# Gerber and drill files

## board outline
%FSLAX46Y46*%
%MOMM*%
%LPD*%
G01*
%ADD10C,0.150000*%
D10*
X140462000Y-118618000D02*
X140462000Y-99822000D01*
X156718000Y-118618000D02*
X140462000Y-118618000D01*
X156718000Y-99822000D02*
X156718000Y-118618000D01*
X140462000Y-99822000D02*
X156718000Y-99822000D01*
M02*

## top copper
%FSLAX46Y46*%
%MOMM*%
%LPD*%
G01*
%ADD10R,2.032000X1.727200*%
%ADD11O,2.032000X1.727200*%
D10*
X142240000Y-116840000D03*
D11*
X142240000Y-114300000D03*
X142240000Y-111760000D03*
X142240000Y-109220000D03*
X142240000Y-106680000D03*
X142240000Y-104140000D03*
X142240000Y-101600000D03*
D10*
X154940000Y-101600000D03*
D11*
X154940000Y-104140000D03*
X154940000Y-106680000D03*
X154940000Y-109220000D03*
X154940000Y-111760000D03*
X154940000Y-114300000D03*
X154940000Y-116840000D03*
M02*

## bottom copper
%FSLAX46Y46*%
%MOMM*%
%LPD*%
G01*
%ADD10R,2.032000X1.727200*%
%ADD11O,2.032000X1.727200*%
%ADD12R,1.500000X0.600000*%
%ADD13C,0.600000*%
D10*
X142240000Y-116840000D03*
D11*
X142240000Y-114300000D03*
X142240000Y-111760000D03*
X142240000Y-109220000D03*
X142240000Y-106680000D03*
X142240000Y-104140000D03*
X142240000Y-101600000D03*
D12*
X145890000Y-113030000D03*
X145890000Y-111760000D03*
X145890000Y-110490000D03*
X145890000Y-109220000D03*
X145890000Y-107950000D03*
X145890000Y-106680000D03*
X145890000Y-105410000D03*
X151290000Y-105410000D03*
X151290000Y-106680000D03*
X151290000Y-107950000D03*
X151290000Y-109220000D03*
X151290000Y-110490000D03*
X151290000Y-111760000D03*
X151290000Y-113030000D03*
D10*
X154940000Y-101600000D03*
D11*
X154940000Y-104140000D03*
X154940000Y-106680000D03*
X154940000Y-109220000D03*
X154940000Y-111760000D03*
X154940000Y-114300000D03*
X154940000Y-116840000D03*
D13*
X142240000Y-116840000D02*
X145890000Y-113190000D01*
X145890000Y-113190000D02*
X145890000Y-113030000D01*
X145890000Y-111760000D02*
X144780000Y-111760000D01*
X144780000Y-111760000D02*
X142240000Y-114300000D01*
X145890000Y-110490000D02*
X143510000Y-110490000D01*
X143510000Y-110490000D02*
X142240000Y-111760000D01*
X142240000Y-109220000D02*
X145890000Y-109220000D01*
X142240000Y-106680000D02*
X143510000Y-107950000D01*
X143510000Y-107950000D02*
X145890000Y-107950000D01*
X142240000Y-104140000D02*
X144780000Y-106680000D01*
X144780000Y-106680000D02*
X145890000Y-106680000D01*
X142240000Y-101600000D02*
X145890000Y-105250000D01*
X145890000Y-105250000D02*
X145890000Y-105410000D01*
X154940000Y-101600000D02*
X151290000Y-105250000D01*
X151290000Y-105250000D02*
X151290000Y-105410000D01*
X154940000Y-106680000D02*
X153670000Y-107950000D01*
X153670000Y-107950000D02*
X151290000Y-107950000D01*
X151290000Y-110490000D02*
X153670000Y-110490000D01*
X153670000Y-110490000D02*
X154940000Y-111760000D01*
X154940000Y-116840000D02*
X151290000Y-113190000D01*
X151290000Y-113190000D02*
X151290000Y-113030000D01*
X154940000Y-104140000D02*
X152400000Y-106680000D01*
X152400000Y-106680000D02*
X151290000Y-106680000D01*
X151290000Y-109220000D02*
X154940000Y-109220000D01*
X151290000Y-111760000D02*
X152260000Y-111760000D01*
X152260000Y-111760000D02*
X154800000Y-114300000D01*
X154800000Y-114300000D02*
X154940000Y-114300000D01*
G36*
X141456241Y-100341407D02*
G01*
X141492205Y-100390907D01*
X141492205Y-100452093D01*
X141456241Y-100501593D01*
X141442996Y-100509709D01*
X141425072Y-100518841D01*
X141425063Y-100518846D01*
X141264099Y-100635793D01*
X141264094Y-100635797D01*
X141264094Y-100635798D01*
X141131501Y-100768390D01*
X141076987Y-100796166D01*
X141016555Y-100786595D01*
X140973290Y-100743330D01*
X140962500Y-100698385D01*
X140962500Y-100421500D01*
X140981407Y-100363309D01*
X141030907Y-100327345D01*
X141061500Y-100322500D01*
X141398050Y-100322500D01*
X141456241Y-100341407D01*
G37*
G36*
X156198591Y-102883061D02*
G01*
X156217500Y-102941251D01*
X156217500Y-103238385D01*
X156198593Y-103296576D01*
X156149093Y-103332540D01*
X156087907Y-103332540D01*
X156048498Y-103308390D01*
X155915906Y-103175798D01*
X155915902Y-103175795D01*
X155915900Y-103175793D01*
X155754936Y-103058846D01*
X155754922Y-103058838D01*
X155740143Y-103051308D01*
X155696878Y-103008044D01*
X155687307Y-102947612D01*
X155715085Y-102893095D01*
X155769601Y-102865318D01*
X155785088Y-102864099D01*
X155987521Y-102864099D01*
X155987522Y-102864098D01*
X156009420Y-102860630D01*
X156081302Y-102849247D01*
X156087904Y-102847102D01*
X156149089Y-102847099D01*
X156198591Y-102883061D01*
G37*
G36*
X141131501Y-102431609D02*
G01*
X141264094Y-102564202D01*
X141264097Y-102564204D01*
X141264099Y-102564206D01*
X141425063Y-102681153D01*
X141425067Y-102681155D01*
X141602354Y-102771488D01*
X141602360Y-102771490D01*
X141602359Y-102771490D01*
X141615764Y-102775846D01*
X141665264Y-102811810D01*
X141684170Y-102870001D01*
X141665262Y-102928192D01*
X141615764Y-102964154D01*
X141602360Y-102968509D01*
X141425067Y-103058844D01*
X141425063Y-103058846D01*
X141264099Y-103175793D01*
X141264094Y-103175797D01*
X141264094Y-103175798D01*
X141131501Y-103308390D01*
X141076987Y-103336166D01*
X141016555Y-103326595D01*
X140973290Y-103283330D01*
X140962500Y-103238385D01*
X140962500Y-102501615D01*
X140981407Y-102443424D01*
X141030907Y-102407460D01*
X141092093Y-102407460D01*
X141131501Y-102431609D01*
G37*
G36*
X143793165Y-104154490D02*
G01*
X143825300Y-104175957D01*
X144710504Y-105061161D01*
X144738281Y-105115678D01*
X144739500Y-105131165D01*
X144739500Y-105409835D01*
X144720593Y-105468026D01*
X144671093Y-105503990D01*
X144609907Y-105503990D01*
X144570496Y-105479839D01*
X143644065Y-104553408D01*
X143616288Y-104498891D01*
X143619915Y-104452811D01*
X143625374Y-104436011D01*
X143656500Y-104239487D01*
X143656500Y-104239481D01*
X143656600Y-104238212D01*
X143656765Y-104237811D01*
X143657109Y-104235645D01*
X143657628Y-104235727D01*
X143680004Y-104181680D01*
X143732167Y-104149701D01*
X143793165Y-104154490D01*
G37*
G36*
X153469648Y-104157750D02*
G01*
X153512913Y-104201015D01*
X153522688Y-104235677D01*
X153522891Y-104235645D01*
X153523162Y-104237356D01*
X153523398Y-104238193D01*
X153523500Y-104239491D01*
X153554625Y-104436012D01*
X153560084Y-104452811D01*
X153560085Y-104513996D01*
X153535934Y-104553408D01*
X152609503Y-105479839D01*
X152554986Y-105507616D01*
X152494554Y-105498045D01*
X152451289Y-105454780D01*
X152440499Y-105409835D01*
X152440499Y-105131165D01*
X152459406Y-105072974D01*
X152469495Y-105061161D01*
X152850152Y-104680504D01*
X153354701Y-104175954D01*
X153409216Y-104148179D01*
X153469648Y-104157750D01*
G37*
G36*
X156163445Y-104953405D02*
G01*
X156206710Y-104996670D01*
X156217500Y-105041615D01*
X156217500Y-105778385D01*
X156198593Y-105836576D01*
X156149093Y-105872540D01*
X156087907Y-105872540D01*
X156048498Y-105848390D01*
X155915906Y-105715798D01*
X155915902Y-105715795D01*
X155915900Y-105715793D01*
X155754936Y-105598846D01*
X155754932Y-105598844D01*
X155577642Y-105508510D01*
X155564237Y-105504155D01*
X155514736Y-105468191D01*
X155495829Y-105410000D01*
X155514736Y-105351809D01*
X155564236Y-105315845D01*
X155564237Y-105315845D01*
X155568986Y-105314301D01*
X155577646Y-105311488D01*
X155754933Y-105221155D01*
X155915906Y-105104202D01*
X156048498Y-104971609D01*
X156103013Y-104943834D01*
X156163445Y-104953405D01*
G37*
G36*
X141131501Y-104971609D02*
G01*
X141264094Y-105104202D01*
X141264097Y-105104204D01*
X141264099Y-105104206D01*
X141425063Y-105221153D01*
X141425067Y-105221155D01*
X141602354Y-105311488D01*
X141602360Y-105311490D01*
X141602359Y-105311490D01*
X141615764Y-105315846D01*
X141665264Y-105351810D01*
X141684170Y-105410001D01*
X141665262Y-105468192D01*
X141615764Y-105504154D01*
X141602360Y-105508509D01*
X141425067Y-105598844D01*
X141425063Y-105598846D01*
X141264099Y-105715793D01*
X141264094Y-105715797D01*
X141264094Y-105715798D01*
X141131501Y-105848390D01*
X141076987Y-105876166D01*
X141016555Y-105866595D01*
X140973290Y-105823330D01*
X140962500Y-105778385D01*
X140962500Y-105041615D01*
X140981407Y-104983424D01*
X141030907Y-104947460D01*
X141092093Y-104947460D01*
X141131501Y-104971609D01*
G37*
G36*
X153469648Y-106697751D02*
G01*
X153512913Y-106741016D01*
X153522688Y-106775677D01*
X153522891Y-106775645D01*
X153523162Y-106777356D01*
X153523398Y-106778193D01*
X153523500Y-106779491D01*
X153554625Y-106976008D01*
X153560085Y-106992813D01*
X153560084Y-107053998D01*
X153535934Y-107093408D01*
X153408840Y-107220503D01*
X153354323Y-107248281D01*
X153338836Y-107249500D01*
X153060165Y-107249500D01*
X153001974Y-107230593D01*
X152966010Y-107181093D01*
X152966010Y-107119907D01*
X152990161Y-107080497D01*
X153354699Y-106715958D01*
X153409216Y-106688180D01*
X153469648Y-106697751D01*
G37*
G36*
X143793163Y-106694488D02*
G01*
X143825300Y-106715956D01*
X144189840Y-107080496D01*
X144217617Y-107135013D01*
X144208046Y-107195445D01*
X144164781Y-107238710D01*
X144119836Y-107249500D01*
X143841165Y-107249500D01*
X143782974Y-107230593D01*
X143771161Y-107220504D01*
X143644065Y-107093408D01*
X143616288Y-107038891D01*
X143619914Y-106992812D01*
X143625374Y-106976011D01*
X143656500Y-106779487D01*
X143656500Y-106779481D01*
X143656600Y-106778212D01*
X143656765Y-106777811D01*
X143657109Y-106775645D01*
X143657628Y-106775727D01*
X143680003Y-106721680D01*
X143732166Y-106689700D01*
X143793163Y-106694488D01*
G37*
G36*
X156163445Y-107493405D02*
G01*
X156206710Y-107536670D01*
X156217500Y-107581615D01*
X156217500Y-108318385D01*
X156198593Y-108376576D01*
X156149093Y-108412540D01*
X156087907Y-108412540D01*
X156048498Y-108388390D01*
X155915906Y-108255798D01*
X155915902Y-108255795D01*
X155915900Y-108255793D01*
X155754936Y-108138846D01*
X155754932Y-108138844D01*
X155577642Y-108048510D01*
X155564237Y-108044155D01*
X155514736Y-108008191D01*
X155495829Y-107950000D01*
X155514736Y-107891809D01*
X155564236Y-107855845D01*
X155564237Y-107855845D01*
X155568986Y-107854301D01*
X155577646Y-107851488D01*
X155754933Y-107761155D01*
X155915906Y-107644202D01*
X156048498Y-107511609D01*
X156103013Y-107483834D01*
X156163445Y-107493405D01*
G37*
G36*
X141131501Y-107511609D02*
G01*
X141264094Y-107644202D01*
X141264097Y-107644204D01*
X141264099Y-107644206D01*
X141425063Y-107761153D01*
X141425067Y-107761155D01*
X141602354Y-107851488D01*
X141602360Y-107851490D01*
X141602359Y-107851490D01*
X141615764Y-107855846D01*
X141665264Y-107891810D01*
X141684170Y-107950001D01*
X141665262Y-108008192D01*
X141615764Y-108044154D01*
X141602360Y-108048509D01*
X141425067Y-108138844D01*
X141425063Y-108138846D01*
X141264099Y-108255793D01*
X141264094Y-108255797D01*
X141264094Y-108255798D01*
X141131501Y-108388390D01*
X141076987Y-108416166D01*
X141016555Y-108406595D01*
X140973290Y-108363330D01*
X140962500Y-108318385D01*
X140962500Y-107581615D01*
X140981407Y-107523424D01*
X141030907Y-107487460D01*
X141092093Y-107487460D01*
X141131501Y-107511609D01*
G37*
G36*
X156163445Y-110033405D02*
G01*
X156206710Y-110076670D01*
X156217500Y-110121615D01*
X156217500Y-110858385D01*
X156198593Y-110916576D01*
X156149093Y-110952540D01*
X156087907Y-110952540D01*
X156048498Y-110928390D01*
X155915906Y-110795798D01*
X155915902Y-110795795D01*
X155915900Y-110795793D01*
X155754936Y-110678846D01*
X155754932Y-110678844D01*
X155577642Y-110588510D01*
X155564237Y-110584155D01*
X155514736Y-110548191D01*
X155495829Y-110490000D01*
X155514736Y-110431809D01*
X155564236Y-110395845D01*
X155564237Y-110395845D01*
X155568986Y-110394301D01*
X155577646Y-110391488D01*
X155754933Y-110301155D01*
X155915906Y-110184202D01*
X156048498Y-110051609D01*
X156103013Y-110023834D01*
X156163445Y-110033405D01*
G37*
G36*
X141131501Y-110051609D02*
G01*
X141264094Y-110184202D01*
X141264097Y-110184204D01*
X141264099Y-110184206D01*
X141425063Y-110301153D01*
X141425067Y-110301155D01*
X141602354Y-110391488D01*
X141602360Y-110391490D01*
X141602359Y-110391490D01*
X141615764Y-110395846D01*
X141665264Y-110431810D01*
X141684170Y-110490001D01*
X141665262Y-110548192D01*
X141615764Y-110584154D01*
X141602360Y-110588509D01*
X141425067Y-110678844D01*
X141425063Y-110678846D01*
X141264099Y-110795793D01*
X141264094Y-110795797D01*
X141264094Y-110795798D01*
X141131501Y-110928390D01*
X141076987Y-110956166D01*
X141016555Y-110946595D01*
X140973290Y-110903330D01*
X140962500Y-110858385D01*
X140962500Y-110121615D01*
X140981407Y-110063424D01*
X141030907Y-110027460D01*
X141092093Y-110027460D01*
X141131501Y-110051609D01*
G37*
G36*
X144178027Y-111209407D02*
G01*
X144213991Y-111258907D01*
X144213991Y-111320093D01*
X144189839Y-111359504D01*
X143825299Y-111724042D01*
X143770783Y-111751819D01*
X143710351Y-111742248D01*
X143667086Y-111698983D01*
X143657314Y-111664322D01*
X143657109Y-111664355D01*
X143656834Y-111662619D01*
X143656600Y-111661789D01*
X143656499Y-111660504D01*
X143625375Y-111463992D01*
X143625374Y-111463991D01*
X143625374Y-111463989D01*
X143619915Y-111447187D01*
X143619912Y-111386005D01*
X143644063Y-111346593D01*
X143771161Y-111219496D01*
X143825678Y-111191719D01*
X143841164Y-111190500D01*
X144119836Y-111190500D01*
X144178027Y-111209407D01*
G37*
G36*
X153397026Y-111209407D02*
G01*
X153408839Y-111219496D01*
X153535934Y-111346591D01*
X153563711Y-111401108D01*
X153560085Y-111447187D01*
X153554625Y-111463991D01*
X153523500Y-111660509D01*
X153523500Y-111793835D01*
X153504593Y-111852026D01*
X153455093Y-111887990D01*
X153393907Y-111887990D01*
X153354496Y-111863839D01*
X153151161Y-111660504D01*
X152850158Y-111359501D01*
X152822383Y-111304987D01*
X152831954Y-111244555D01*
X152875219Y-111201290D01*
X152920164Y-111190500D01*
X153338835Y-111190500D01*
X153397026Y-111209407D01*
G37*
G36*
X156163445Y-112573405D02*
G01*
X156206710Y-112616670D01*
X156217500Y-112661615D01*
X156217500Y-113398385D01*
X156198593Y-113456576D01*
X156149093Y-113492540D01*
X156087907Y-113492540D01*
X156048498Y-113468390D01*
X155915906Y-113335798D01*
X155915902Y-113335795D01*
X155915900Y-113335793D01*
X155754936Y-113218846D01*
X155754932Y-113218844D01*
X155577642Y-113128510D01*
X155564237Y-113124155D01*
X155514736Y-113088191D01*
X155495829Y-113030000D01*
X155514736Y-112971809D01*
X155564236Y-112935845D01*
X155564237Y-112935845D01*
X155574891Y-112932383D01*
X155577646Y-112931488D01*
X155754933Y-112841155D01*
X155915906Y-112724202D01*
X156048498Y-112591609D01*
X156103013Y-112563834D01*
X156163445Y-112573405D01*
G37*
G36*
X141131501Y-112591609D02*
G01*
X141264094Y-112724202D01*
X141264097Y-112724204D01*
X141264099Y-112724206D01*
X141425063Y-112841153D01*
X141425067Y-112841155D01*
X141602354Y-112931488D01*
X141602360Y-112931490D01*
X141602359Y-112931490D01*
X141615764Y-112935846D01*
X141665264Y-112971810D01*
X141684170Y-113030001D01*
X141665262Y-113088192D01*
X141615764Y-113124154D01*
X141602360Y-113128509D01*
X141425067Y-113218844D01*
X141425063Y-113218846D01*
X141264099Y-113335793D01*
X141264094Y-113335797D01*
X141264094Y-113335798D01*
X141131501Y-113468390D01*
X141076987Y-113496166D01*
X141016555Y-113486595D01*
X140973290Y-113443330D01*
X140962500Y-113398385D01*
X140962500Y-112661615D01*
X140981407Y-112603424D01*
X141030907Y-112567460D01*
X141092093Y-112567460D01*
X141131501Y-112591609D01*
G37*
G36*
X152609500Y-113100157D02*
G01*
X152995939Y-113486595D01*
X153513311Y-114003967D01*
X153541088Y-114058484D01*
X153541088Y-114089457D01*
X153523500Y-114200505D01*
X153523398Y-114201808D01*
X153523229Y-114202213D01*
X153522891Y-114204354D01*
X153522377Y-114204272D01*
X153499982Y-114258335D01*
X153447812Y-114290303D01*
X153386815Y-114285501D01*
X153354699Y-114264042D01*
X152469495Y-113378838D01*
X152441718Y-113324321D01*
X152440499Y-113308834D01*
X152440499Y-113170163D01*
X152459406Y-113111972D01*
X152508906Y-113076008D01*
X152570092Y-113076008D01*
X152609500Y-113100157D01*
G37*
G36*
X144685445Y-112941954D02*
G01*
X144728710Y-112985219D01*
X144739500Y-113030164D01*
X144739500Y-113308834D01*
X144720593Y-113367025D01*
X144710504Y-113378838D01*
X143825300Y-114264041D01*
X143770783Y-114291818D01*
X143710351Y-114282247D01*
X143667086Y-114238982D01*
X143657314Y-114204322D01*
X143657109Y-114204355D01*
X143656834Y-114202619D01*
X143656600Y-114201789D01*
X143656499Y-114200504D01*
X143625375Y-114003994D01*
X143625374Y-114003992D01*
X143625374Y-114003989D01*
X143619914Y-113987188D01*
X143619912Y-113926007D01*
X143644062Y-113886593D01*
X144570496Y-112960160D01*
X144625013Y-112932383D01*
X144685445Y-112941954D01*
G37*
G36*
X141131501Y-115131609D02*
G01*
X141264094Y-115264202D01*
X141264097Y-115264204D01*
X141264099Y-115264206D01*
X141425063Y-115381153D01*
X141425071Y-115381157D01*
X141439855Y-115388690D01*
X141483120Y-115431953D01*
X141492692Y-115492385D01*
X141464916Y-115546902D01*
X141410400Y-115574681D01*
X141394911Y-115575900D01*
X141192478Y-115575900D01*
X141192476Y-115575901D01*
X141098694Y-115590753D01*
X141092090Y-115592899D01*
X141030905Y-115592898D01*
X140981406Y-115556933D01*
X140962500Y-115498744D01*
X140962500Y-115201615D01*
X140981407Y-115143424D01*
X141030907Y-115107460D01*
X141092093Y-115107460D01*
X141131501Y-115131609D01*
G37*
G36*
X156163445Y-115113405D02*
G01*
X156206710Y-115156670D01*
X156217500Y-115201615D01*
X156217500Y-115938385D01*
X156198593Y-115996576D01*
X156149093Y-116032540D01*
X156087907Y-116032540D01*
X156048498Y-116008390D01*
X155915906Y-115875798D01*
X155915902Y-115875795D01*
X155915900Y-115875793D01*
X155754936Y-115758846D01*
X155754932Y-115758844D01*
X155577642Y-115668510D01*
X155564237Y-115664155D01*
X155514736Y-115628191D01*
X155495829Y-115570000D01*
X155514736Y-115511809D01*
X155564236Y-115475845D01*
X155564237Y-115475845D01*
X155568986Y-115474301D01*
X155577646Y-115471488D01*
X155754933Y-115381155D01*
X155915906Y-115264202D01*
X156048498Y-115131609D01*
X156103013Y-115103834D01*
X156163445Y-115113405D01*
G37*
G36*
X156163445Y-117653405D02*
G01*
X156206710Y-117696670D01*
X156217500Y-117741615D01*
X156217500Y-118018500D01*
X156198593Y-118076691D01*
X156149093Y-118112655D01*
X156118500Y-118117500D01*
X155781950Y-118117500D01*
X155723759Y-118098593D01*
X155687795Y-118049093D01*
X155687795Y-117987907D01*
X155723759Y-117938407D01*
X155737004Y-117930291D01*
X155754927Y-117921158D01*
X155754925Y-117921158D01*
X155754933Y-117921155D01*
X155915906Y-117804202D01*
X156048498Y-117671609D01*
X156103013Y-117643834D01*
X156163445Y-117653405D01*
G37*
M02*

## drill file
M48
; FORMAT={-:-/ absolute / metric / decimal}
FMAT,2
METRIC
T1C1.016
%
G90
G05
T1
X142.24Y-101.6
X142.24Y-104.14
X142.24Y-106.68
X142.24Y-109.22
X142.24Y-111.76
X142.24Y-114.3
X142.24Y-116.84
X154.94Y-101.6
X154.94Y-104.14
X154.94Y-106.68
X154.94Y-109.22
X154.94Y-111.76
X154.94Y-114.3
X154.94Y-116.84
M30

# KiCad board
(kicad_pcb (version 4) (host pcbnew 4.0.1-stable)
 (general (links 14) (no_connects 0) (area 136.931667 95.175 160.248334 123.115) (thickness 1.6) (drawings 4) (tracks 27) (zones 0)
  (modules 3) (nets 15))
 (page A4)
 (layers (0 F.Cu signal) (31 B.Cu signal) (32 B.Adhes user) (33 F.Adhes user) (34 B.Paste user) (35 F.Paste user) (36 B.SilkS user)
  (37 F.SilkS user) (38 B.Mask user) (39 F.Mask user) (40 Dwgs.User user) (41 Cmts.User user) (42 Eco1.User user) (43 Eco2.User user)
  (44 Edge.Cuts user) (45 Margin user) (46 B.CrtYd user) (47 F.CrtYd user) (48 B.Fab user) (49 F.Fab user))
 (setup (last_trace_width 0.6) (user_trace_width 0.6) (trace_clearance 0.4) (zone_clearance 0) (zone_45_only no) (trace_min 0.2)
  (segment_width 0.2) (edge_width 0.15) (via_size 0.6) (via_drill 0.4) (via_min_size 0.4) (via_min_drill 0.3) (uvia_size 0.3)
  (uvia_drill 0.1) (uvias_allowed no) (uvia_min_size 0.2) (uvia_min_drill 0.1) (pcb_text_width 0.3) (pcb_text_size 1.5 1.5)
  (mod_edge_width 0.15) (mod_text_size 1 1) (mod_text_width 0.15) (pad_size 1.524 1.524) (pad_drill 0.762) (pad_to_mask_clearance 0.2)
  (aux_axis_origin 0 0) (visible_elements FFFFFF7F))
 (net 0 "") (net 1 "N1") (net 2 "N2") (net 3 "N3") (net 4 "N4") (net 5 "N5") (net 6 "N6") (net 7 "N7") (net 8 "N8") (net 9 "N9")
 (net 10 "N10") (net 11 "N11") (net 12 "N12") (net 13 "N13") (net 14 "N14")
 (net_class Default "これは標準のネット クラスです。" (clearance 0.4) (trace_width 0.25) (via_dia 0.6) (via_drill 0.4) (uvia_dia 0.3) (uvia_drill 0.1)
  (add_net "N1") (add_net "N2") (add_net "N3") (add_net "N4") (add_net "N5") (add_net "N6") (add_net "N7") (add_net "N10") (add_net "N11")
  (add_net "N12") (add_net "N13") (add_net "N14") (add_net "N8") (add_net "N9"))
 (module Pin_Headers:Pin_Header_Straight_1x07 (layer F.Cu) (at 142.24 116.84 180)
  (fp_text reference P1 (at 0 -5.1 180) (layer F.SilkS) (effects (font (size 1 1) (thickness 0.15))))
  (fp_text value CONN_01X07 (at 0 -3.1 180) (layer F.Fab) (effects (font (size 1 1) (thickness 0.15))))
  (pad 1 thru_hole rect (at 0 0 180) (size 2.032 1.7272) (drill 1.016) (layers *.Cu *.Mask F.SilkS) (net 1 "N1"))
  (pad 2 thru_hole oval (at 0 2.54 180) (size 2.032 1.7272) (drill 1.016) (layers *.Cu *.Mask F.SilkS) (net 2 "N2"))
  (pad 3 thru_hole oval (at 0 5.08 180) (size 2.032 1.7272) (drill 1.016) (layers *.Cu *.Mask F.SilkS) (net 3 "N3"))
  (pad 4 thru_hole oval (at 0 7.62 180) (size 2.032 1.7272) (drill 1.016) (layers *.Cu *.Mask F.SilkS) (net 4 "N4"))
  (pad 5 thru_hole oval (at 0 10.16 180) (size 2.032 1.7272) (drill 1.016) (layers *.Cu *.Mask F.SilkS) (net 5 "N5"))
  (pad 6 thru_hole oval (at 0 12.7 180) (size 2.032 1.7272) (drill 1.016) (layers *.Cu *.Mask F.SilkS) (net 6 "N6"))
  (pad 7 thru_hole oval (at 0 15.24 180) (size 2.032 1.7272) (drill 1.016) (layers *.Cu *.Mask F.SilkS) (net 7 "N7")))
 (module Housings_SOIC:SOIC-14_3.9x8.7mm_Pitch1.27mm (layer B.Cu) (at 148.59 109.22)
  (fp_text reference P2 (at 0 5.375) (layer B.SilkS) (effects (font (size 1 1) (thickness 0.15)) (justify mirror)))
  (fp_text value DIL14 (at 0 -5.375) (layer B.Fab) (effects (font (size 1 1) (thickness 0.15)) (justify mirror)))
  (pad 1 smd rect (at -2.7 3.81) (size 1.5 0.6) (layers B.Cu B.Paste B.Mask) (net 1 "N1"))
  (pad 2 smd rect (at -2.7 2.54) (size 1.5 0.6) (layers B.Cu B.Paste B.Mask) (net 2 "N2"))
  (pad 3 smd rect (at -2.7 1.27) (size 1.5 0.6) (layers B.Cu B.Paste B.Mask) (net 3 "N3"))
  (pad 4 smd rect (at -2.7 0) (size 1.5 0.6) (layers B.Cu B.Paste B.Mask) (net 4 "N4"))
  (pad 5 smd rect (at -2.7 -1.27) (size 1.5 0.6) (layers B.Cu B.Paste B.Mask) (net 5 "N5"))
  (pad 6 smd rect (at -2.7 -2.54) (size 1.5 0.6) (layers B.Cu B.Paste B.Mask) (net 6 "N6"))
  (pad 7 smd rect (at -2.7 -3.81) (size 1.5 0.6) (layers B.Cu B.Paste B.Mask) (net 7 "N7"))
  (pad 8 smd rect (at 2.7 -3.81) (size 1.5 0.6) (layers B.Cu B.Paste B.Mask) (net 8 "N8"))
  (pad 9 smd rect (at 2.7 -2.54) (size 1.5 0.6) (layers B.Cu B.Paste B.Mask) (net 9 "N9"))
  (pad 10 smd rect (at 2.7 -1.27) (size 1.5 0.6) (layers B.Cu B.Paste B.Mask) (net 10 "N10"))
  (pad 11 smd rect (at 2.7 0) (size 1.5 0.6) (layers B.Cu B.Paste B.Mask) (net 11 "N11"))
  (pad 12 smd rect (at 2.7 1.27) (size 1.5 0.6) (layers B.Cu B.Paste B.Mask) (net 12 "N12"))
  (pad 13 smd rect (at 2.7 2.54) (size 1.5 0.6) (layers B.Cu B.Paste B.Mask) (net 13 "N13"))
  (pad 14 smd rect (at 2.7 3.81) (size 1.5 0.6) (layers B.Cu B.Paste B.Mask) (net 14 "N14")))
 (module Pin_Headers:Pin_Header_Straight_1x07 (layer F.Cu) (at 154.94 101.6)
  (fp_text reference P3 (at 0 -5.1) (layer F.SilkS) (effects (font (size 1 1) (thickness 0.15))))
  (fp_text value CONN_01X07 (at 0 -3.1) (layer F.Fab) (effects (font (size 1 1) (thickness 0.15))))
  (pad 1 thru_hole rect (at 0 0) (size 2.032 1.7272) (drill 1.016) (layers *.Cu *.Mask F.SilkS) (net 8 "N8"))
  (pad 2 thru_hole oval (at 0 2.54) (size 2.032 1.7272) (drill 1.016) (layers *.Cu *.Mask F.SilkS) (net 9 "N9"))
  (pad 3 thru_hole oval (at 0 5.08) (size 2.032 1.7272) (drill 1.016) (layers *.Cu *.Mask F.SilkS) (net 10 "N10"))
  (pad 4 thru_hole oval (at 0 7.62) (size 2.032 1.7272) (drill 1.016) (layers *.Cu *.Mask F.SilkS) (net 11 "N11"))
  (pad 5 thru_hole oval (at 0 10.16) (size 2.032 1.7272) (drill 1.016) (layers *.Cu *.Mask F.SilkS) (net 12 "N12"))
  (pad 6 thru_hole oval (at 0 12.7) (size 2.032 1.7272) (drill 1.016) (layers *.Cu *.Mask F.SilkS) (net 13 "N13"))
  (pad 7 thru_hole oval (at 0 15.24) (size 2.032 1.7272) (drill 1.016) (layers *.Cu *.Mask F.SilkS) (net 14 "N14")))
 (gr_line (start 140.462 118.618) (end 140.462 99.822) (angle 90) (layer Edge.Cuts) (width 0.15))
 (gr_line (start 156.718 118.618) (end 140.462 118.618) (angle 90) (layer Edge.Cuts) (width 0.15))
 (gr_line (start 156.718 99.822) (end 156.718 118.618) (angle 90) (layer Edge.Cuts) (width 0.15))
 (gr_line (start 140.462 99.822) (end 156.718 99.822) (angle 90) (layer Edge.Cuts) (width 0.15))
 (segment (start 142.24 116.84) (end 145.89 113.19) (width 0.6) (layer B.Cu) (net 1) (status C00000))
 (segment (start 145.89 113.19) (end 145.89 113.03) (width 0.6) (layer B.Cu) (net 1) (status C00000))
 (segment (start 145.89 111.76) (end 144.78 111.76) (width 0.6) (layer B.Cu) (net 2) (status 400000))
 (segment (start 144.78 111.76) (end 142.24 114.3) (width 0.6) (layer B.Cu) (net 2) (status 800000))
 (segment (start 145.89 110.49) (end 143.51 110.49) (width 0.6) (layer B.Cu) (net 3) (status 400000))
 (segment (start 143.51 110.49) (end 142.24 111.76) (width 0.6) (layer B.Cu) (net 3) (status 800000))
 (segment (start 142.24 109.22) (end 145.89 109.22) (width 0.6) (layer B.Cu) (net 4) (status C00000))
 (segment (start 142.24 106.68) (end 143.51 107.95) (width 0.6) (layer B.Cu) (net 5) (status 400000))
 (segment (start 143.51 107.95) (end 145.89 107.95) (width 0.6) (layer B.Cu) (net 5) (status 800000))
 (segment (start 142.24 104.14) (end 144.78 106.68) (width 0.6) (layer B.Cu) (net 6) (status 400000))
 (segment (start 144.78 106.68) (end 145.89 106.68) (width 0.6) (layer B.Cu) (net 6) (status 800000))
 (segment (start 142.24 101.6) (end 145.89 105.25) (width 0.6) (layer B.Cu) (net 7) (status C00000))
 (segment (start 145.89 105.25) (end 145.89 105.41) (width 0.6) (layer B.Cu) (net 7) (status C00000))
 (segment (start 154.94 101.6) (end 151.29 105.25) (width 0.6) (layer B.Cu) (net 8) (status C00000))
 (segment (start 151.29 105.25) (end 151.29 105.41) (width 0.6) (layer B.Cu) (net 8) (status C00000))
 (segment (start 154.94 106.68) (end 153.67 107.95) (width 0.6) (layer B.Cu) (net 10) (status 400000))
 (segment (start 153.67 107.95) (end 151.29 107.95) (width 0.6) (layer B.Cu) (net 10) (status 800000))
 (segment (start 151.29 110.49) (end 153.67 110.49) (width 0.6) (layer B.Cu) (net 12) (status 400000))
 (segment (start 153.67 110.49) (end 154.94 111.76) (width 0.6) (layer B.Cu) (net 12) (status 800000))
 (segment (start 154.94 116.84) (end 151.29 113.19) (width 0.6) (layer B.Cu) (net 14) (status C00000))
 (segment (start 151.29 113.19) (end 151.29 113.03) (width 0.6) (layer B.Cu) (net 14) (status C00000))
 (segment (start 154.94 104.14) (end 152.4 106.68) (width 0.6) (layer B.Cu) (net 9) (status 400000))
 (segment (start 152.4 106.68) (end 151.29 106.68) (width 0.6) (layer B.Cu) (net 9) (status 800000))
 (segment (start 151.29 109.22) (end 154.94 109.22) (width 0.6) (layer B.Cu) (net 11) (status C00000))
 (segment (start 151.29 111.76) (end 152.26 111.76) (width 0.6) (layer B.Cu) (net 13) (status 400000))
 (segment (start 152.26 111.76) (end 154.8 114.3) (width 0.6) (layer B.Cu) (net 13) (status 800000))
 (segment (start 154.8 114.3) (end 154.94 114.3) (width 0.6) (layer B.Cu) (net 13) (status C00000))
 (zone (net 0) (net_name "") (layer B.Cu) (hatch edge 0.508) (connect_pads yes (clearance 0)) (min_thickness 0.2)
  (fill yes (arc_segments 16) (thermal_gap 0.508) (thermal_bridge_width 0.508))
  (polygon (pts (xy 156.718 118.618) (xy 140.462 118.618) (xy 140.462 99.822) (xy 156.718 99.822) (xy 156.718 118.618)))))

